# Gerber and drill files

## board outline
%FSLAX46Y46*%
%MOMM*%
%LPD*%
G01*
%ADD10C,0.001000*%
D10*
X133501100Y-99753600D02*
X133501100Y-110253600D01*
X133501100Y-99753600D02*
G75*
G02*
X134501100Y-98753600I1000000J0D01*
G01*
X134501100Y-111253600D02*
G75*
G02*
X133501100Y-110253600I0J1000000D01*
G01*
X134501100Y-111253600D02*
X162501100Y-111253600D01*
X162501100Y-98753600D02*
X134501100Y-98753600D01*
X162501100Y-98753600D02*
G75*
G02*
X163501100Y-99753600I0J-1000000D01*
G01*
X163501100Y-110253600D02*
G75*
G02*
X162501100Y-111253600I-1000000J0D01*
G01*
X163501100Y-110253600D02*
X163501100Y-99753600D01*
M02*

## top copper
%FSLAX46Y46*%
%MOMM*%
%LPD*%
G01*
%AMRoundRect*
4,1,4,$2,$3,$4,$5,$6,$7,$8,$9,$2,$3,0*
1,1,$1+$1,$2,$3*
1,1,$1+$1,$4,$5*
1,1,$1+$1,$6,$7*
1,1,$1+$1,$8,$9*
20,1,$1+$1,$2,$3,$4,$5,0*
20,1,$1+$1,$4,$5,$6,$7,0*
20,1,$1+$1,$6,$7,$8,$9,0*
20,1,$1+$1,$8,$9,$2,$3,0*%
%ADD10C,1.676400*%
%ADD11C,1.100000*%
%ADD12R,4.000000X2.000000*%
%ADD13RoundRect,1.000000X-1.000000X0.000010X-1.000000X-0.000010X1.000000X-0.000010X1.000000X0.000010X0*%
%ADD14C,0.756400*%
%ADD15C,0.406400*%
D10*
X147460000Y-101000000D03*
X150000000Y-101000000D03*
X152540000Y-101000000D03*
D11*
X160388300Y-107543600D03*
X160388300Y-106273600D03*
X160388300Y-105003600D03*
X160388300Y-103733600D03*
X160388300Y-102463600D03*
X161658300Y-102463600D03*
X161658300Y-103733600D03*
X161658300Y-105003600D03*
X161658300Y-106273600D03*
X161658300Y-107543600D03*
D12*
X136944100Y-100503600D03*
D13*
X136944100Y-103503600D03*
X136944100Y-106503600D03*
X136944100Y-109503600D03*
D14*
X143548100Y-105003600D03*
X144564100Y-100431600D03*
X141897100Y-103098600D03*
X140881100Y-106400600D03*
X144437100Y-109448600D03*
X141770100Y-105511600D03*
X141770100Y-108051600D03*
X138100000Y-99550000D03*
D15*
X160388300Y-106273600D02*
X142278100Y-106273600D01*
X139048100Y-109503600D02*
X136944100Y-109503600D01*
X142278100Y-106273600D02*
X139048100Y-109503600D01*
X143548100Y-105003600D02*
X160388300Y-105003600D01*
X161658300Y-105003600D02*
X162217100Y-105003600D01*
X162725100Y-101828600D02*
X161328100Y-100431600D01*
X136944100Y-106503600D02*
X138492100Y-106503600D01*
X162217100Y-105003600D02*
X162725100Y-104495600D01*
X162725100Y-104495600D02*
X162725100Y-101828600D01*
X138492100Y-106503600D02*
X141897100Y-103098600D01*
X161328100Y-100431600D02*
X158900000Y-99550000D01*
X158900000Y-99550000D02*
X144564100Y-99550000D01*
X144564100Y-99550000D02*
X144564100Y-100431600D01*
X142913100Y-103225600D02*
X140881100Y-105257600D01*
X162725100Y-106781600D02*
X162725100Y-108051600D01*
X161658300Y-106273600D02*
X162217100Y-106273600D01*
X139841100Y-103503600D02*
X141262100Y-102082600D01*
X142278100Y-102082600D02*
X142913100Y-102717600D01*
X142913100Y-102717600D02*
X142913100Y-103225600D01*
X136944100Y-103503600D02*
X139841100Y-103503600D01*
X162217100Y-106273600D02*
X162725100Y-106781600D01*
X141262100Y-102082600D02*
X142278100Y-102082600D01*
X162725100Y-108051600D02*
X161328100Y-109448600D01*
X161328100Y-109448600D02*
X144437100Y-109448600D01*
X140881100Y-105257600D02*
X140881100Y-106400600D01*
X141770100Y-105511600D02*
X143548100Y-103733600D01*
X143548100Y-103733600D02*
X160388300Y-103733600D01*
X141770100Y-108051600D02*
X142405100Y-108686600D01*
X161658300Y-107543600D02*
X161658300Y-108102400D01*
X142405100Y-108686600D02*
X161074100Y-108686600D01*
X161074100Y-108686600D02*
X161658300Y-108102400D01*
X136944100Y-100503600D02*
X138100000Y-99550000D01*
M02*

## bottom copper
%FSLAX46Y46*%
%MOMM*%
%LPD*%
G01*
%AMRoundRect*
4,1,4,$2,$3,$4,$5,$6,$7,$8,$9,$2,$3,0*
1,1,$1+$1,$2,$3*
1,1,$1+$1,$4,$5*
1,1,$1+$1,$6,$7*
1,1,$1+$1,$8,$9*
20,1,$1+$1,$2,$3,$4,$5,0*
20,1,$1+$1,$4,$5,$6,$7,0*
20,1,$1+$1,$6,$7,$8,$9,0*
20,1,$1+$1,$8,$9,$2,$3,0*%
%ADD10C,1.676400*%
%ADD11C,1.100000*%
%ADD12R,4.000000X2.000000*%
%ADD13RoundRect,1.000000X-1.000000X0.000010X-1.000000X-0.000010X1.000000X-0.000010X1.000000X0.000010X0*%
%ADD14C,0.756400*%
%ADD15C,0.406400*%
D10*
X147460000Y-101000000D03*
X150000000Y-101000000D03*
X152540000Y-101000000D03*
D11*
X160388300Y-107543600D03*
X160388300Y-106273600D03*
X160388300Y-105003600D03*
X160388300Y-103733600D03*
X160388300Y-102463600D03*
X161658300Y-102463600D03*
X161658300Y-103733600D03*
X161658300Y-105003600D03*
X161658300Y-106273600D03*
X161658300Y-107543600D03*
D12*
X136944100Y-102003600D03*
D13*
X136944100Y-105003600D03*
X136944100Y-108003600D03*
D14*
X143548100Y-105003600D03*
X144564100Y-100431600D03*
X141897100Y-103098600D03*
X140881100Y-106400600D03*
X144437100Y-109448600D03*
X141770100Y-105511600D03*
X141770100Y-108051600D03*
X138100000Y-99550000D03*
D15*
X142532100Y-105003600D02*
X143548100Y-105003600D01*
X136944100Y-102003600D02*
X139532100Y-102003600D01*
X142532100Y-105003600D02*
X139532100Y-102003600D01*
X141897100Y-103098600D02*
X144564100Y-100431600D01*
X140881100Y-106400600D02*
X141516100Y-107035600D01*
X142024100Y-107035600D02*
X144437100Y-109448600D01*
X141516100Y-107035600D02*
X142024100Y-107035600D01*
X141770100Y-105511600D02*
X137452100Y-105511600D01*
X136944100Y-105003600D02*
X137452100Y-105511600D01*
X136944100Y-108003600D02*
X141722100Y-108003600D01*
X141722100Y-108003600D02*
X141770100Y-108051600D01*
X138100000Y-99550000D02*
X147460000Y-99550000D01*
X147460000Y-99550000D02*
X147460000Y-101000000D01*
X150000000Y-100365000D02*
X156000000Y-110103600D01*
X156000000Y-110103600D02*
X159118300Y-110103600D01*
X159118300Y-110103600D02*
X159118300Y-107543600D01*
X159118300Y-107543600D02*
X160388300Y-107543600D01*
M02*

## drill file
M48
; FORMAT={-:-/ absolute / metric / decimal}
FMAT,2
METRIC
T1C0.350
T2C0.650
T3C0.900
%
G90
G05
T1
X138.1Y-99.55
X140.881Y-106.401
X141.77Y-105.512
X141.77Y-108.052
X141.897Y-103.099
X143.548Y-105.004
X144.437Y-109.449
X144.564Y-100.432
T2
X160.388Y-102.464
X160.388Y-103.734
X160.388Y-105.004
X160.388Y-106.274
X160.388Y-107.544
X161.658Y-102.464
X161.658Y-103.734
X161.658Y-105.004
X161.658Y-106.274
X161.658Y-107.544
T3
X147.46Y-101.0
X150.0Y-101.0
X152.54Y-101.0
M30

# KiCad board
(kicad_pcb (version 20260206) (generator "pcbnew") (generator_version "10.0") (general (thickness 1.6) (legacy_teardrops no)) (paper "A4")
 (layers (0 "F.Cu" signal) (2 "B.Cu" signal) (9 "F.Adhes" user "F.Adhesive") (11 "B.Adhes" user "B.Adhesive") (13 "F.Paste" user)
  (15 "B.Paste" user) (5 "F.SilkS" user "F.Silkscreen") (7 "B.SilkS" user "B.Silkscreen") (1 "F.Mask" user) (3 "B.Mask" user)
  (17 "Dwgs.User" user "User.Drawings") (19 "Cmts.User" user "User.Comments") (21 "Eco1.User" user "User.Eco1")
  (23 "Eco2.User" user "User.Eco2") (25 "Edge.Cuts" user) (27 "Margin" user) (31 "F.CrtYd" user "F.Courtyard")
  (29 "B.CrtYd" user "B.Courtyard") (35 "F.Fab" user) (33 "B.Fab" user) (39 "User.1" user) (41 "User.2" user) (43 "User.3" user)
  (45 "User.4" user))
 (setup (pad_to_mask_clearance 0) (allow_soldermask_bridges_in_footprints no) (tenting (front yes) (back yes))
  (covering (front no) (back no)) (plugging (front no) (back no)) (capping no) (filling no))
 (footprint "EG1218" (layer "F.Cu") (at 150 101)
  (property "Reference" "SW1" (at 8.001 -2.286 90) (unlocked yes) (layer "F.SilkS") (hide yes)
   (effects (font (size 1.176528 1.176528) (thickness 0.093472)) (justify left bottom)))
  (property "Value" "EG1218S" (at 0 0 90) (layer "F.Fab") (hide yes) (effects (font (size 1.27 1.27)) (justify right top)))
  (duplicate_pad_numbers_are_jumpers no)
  (pad "O" thru_hole circle (at -2.54 0 90) (size 1.6764 1.6764) (drill 0.9) (layers "*.Cu" "*.Mask") (remove_unused_layers no)
   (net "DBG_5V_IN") (solder_mask_margin 0.1016) (thermal_bridge_angle 0))
  (pad "P" thru_hole circle (at 0 0 90) (size 1.6764 1.6764) (drill 0.9) (layers "*.Cu" "*.Mask") (remove_unused_layers no) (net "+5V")
   (solder_mask_margin 0.1016) (thermal_bridge_angle 0))
  (pad "S" thru_hole circle (at 2.54 0 90) (size 1.6764 1.6764) (drill 0.9) (layers "*.Cu" "*.Mask") (remove_unused_layers no)
   (solder_mask_margin 0.1016) (thermal_bridge_angle 0)))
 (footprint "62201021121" (layer "F.Cu") (at 161.0233 105.0036 90)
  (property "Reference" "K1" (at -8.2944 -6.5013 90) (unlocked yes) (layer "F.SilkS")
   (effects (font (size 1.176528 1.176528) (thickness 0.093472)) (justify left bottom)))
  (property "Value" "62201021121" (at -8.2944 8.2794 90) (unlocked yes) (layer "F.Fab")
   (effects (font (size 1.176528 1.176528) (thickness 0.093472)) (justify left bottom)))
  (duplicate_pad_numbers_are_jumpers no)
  (pad "1" thru_hole circle (at -2.54 -0.635 90) (size 1.1 1.1) (drill 0.65) (layers "*.Cu" "*.Mask") (remove_unused_layers no) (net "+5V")
   (solder_mask_margin 0.1016) (thermal_bridge_angle 0))
  (pad "2" thru_hole circle (at -1.27 -0.635 90) (size 1.1 1.1) (drill 0.65) (layers "*.Cu" "*.Mask") (remove_unused_layers no) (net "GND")
   (solder_mask_margin 0.1016) (thermal_bridge_angle 0))
  (pad "3" thru_hole circle (at 0 -0.635 90) (size 1.1 1.1) (drill 0.65) (layers "*.Cu" "*.Mask") (remove_unused_layers no) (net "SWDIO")
   (solder_mask_margin 0.1016) (thermal_bridge_angle 0))
  (pad "4" thru_hole circle (at 1.27 -0.635 90) (size 1.1 1.1) (drill 0.65) (layers "*.Cu" "*.Mask") (remove_unused_layers no) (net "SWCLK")
   (solder_mask_margin 0.1016) (thermal_bridge_angle 0))
  (pad "5" thru_hole circle (at 2.54 -0.635 90) (size 1.1 1.1) (drill 0.65) (layers "*.Cu" "*.Mask") (remove_unused_layers no) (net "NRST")
   (solder_mask_margin 0.1016) (thermal_bridge_angle 0))
  (pad "6" thru_hole circle (at 2.54 0.635 90) (size 1.1 1.1) (drill 0.65) (layers "*.Cu" "*.Mask") (remove_unused_layers no) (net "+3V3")
   (solder_mask_margin 0.1016) (thermal_bridge_angle 0))
  (pad "7" thru_hole circle (at 1.27 0.635 90) (size 1.1 1.1) (drill 0.65) (layers "*.Cu" "*.Mask") (remove_unused_layers no) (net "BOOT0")
   (solder_mask_margin 0.1016) (thermal_bridge_angle 0))
  (pad "8" thru_hole circle (at 0 0.635 90) (size 1.1 1.1) (drill 0.65) (layers "*.Cu" "*.Mask") (remove_unused_layers no) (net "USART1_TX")
   (solder_mask_margin 0.1016) (thermal_bridge_angle 0))
  (pad "9" thru_hole circle (at -1.27 0.635 90) (size 1.1 1.1) (drill 0.65) (layers "*.Cu" "*.Mask") (remove_unused_layers no)
   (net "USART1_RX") (solder_mask_margin 0.1016) (thermal_bridge_angle 0))
  (pad "10" thru_hole circle (at -2.54 0.635 90) (size 1.1 1.1) (drill 0.65) (layers "*.Cu" "*.Mask") (remove_unused_layers no) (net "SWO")
   (solder_mask_margin 0.1016) (thermal_bridge_angle 0)))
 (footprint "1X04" (layer "F.Cu") (at 136.9441 105.0036 -90)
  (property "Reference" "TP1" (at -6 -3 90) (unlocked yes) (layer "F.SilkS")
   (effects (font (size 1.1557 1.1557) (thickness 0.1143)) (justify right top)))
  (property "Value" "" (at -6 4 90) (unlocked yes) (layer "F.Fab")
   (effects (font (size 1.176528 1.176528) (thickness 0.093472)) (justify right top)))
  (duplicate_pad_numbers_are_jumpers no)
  (pad "1" smd rect (at -4.5 0 270) (size 2 4) (layers "F.Cu" "F.Mask" "F.Paste") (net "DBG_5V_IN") (solder_mask_margin 0.1016)
   (solder_paste_margin 0) (thermal_bridge_angle 0))
  (pad "2" smd roundrect (at -1.5 0 270) (size 2 4) (layers "F.Cu" "F.Mask" "F.Paste") (roundrect_rratio 0.5) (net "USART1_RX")
   (solder_mask_margin 0.1016) (solder_paste_margin 0) (thermal_bridge_angle 0))
  (pad "3" smd roundrect (at 1.5 0 270) (size 2 4) (layers "F.Cu" "F.Mask" "F.Paste") (roundrect_rratio 0.5) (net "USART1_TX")
   (solder_mask_margin 0.1016) (solder_paste_margin 0) (thermal_bridge_angle 0))
  (pad "4" smd roundrect (at 4.5 0 270) (size 2 4) (layers "F.Cu" "F.Mask" "F.Paste") (roundrect_rratio 0.5) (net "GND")
   (solder_mask_margin 0.1016) (solder_paste_margin 0) (thermal_bridge_angle 0)))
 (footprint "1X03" (layer "B.Cu") (at 136.9441 105.0036 -90)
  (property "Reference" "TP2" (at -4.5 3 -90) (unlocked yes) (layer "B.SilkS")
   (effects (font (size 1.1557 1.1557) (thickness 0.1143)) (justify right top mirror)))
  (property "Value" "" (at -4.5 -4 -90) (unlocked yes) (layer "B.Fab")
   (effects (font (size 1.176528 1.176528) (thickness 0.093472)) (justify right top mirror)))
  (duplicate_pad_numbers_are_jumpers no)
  (pad "1" smd rect (at -3 0 270) (size 2 4) (layers "B.Cu" "B.Mask" "B.Paste") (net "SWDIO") (solder_mask_margin 0.1016)
   (solder_paste_margin 0) (thermal_bridge_angle 0))
  (pad "2" smd roundrect (at 0 0 270) (size 2 4) (layers "B.Cu" "B.Mask" "B.Paste") (roundrect_rratio 0.5) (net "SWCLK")
   (solder_mask_margin 0.1016) (solder_paste_margin 0) (thermal_bridge_angle 0))
  (pad "3" smd roundrect (at 3 0 270) (size 2 4) (layers "B.Cu" "B.Mask" "B.Paste") (roundrect_rratio 0.5) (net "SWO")
   (solder_mask_margin 0.1016) (solder_paste_margin 0) (thermal_bridge_angle 0)))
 (gr_line (start 133.5011 99.7536) (end 133.5011 110.2536) (stroke (width 0.001) (type solid)) (layer "Edge.Cuts"))
 (gr_arc (start 133.5011 99.7536) (mid 133.793993 99.046493) (end 134.5011 98.7536) (stroke (width 0.001) (type solid)) (layer "Edge.Cuts"))
 (gr_arc (start 134.5011 111.2536) (mid 133.793993 110.960707) (end 133.5011 110.2536) (stroke (width 0.001) (type solid))
  (layer "Edge.Cuts"))
 (gr_line (start 134.5011 111.2536) (end 162.5011 111.2536) (stroke (width 0.001) (type solid)) (layer "Edge.Cuts"))
 (gr_line (start 162.5011 98.7536) (end 134.5011 98.7536) (stroke (width 0.001) (type solid)) (layer "Edge.Cuts"))
 (gr_arc (start 162.5011 98.7536) (mid 163.208207 99.046493) (end 163.5011 99.7536) (stroke (width 0.001) (type solid)) (layer "Edge.Cuts"))
 (gr_arc (start 163.5011 110.2536) (mid 163.208207 110.960707) (end 162.5011 111.2536) (stroke (width 0.001) (type solid))
  (layer "Edge.Cuts"))
 (gr_line (start 163.5011 110.2536) (end 163.5011 99.7536) (stroke (width 0.001) (type solid)) (layer "Edge.Cuts"))
 (segment (start 160.3883 106.2736) (end 142.2781 106.2736) (width 0.4064) (layer "F.Cu") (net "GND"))
 (segment (start 139.0481 109.5036) (end 136.9441 109.5036) (width 0.4064) (layer "F.Cu") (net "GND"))
 (segment (start 142.2781 106.2736) (end 139.0481 109.5036) (width 0.4064) (layer "F.Cu") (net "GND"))
 (segment (start 143.5481 105.0036) (end 160.3883 105.0036) (width 0.4064) (layer "F.Cu") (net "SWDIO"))
 (via (at 143.5481 105.0036) (size 0.7564) (drill 0.35) (layers "F.Cu" "B.Cu") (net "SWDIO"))
 (segment (start 142.5321 105.0036) (end 143.5481 105.0036) (width 0.4064) (layer "B.Cu") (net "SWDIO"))
 (segment (start 136.9441 102.0036) (end 139.5321 102.0036) (width 0.4064) (layer "B.Cu") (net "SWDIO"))
 (segment (start 142.5321 105.0036) (end 139.5321 102.0036) (width 0.4064) (layer "B.Cu") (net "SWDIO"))
 (segment (start 161.6583 105.0036) (end 162.2171 105.0036) (width 0.4064) (layer "F.Cu") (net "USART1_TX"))
 (segment (start 162.7251 101.8286) (end 161.3281 100.4316) (width 0.4064) (layer "F.Cu") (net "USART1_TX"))
 (segment (start 136.9441 106.5036) (end 138.4921 106.5036) (width 0.4064) (layer "F.Cu") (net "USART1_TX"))
 (segment (start 162.2171 105.0036) (end 162.7251 104.4956) (width 0.4064) (layer "F.Cu") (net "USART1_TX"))
 (segment (start 162.7251 104.4956) (end 162.7251 101.8286) (width 0.4064) (layer "F.Cu") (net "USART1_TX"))
 (segment (start 138.4921 106.5036) (end 141.8971 103.0986) (width 0.4064) (layer "F.Cu") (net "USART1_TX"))
 (segment (start 161.3281 100.4316) (end 158.9 99.55) (width 0.4064) (layer "F.Cu") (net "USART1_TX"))
 (segment (start 158.9 99.55) (end 144.5641 99.55) (width 0.4064) (layer "F.Cu") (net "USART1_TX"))
 (segment (start 144.5641 99.55) (end 144.5641 100.4316) (width 0.4064) (layer "F.Cu") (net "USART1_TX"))
 (via (at 144.5641 100.4316) (size 0.7564) (drill 0.35) (layers "F.Cu" "B.Cu") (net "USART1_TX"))
 (via (at 141.8971 103.0986) (size 0.7564) (drill 0.35) (layers "F.Cu" "B.Cu") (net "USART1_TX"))
 (segment (start 141.8971 103.0986) (end 144.5641 100.4316) (width 0.4064) (layer "B.Cu") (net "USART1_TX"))
 (segment (start 142.9131 103.2256) (end 140.8811 105.2576) (width 0.4064) (layer "F.Cu") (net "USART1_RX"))
 (segment (start 162.7251 106.7816) (end 162.7251 108.0516) (width 0.4064) (layer "F.Cu") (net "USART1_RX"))
 (segment (start 161.6583 106.2736) (end 162.2171 106.2736) (width 0.4064) (layer "F.Cu") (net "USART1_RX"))
 (segment (start 139.8411 103.5036) (end 141.2621 102.0826) (width 0.4064) (layer "F.Cu") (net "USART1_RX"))
 (segment (start 142.2781 102.0826) (end 142.9131 102.7176) (width 0.4064) (layer "F.Cu") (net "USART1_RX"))
 (segment (start 142.9131 102.7176) (end 142.9131 103.2256) (width 0.4064) (layer "F.Cu") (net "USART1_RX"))
 (segment (start 136.9441 103.5036) (end 139.8411 103.5036) (width 0.4064) (layer "F.Cu") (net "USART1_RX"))
 (segment (start 162.2171 106.2736) (end 162.7251 106.7816) (width 0.4064) (layer "F.Cu") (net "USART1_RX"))
 (segment (start 141.2621 102.0826) (end 142.2781 102.0826) (width 0.4064) (layer "F.Cu") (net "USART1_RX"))
 (segment (start 162.7251 108.0516) (end 161.3281 109.4486) (width 0.4064) (layer "F.Cu") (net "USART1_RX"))
 (segment (start 161.3281 109.4486) (end 144.4371 109.4486) (width 0.4064) (layer "F.Cu") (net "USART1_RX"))
 (segment (start 140.8811 105.2576) (end 140.8811 106.4006) (width 0.4064) (layer "F.Cu") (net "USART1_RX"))
 (via (at 140.8811 106.4006) (size 0.7564) (drill 0.35) (layers "F.Cu" "B.Cu") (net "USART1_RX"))
 (via (at 144.4371 109.4486) (size 0.7564) (drill 0.35) (layers "F.Cu" "B.Cu") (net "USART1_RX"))
 (segment (start 140.8811 106.4006) (end 141.5161 107.0356) (width 0.4064) (layer "B.Cu") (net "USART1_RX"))
 (segment (start 142.0241 107.0356) (end 144.4371 109.4486) (width 0.4064) (layer "B.Cu") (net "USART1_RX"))
 (segment (start 141.5161 107.0356) (end 142.0241 107.0356) (width 0.4064) (layer "B.Cu") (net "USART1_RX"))
 (segment (start 141.7701 105.5116) (end 143.5481 103.7336) (width 0.4064) (layer "F.Cu") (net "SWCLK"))
 (segment (start 143.5481 103.7336) (end 160.3883 103.7336) (width 0.4064) (layer "F.Cu") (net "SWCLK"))
 (via (at 141.7701 105.5116) (size 0.7564) (drill 0.35) (layers "F.Cu" "B.Cu") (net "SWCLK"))
 (segment (start 141.7701 105.5116) (end 137.4521 105.5116) (width 0.4064) (layer "B.Cu") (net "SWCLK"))
 (segment (start 136.9441 105.0036) (end 137.4521 105.5116) (width 0.4064) (layer "B.Cu") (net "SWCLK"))
 (segment (start 141.7701 108.0516) (end 142.4051 108.6866) (width 0.4064) (layer "F.Cu") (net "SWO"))
 (segment (start 161.6583 107.5436) (end 161.6583 108.1024) (width 0.4064) (layer "F.Cu") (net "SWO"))
 (segment (start 142.4051 108.6866) (end 161.0741 108.6866) (width 0.4064) (layer "F.Cu") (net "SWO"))
 (segment (start 161.0741 108.6866) (end 161.6583 108.1024) (width 0.4064) (layer "F.Cu") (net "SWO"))
 (via (at 141.7701 108.0516) (size 0.7564) (drill 0.35) (layers "F.Cu" "B.Cu") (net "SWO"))
 (segment (start 136.9441 108.0036) (end 141.7221 108.0036) (width 0.4064) (layer "B.Cu") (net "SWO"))
 (segment (start 141.7221 108.0036) (end 141.7701 108.0516) (width 0.4064) (layer "B.Cu") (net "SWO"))
 (segment (start 136.9441 100.5036) (end 138.1 99.55) (width 0.4064) (layer "F.Cu") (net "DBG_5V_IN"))
 (via (at 138.1 99.55) (size 0.7564) (drill 0.35) (layers "F.Cu" "B.Cu") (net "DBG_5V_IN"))
 (segment (start 138.1 99.55) (end 147.46 99.55) (width 0.4064) (layer "B.Cu") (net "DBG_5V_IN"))
 (segment (start 147.46 99.55) (end 147.46 101) (width 0.4064) (layer "B.Cu") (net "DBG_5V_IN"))
 (segment (start 150 100.365) (end 156 110.1036) (width 0.4064) (layer "B.Cu") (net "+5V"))
 (segment (start 156 110.1036) (end 159.1183 110.1036) (width 0.4064) (layer "B.Cu") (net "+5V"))
 (segment (start 159.1183 110.1036) (end 159.1183 107.5436) (width 0.4064) (layer "B.Cu") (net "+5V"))
 (segment (start 159.1183 107.5436) (end 160.3883 107.5436) (width 0.4064) (layer "B.Cu") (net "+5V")))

